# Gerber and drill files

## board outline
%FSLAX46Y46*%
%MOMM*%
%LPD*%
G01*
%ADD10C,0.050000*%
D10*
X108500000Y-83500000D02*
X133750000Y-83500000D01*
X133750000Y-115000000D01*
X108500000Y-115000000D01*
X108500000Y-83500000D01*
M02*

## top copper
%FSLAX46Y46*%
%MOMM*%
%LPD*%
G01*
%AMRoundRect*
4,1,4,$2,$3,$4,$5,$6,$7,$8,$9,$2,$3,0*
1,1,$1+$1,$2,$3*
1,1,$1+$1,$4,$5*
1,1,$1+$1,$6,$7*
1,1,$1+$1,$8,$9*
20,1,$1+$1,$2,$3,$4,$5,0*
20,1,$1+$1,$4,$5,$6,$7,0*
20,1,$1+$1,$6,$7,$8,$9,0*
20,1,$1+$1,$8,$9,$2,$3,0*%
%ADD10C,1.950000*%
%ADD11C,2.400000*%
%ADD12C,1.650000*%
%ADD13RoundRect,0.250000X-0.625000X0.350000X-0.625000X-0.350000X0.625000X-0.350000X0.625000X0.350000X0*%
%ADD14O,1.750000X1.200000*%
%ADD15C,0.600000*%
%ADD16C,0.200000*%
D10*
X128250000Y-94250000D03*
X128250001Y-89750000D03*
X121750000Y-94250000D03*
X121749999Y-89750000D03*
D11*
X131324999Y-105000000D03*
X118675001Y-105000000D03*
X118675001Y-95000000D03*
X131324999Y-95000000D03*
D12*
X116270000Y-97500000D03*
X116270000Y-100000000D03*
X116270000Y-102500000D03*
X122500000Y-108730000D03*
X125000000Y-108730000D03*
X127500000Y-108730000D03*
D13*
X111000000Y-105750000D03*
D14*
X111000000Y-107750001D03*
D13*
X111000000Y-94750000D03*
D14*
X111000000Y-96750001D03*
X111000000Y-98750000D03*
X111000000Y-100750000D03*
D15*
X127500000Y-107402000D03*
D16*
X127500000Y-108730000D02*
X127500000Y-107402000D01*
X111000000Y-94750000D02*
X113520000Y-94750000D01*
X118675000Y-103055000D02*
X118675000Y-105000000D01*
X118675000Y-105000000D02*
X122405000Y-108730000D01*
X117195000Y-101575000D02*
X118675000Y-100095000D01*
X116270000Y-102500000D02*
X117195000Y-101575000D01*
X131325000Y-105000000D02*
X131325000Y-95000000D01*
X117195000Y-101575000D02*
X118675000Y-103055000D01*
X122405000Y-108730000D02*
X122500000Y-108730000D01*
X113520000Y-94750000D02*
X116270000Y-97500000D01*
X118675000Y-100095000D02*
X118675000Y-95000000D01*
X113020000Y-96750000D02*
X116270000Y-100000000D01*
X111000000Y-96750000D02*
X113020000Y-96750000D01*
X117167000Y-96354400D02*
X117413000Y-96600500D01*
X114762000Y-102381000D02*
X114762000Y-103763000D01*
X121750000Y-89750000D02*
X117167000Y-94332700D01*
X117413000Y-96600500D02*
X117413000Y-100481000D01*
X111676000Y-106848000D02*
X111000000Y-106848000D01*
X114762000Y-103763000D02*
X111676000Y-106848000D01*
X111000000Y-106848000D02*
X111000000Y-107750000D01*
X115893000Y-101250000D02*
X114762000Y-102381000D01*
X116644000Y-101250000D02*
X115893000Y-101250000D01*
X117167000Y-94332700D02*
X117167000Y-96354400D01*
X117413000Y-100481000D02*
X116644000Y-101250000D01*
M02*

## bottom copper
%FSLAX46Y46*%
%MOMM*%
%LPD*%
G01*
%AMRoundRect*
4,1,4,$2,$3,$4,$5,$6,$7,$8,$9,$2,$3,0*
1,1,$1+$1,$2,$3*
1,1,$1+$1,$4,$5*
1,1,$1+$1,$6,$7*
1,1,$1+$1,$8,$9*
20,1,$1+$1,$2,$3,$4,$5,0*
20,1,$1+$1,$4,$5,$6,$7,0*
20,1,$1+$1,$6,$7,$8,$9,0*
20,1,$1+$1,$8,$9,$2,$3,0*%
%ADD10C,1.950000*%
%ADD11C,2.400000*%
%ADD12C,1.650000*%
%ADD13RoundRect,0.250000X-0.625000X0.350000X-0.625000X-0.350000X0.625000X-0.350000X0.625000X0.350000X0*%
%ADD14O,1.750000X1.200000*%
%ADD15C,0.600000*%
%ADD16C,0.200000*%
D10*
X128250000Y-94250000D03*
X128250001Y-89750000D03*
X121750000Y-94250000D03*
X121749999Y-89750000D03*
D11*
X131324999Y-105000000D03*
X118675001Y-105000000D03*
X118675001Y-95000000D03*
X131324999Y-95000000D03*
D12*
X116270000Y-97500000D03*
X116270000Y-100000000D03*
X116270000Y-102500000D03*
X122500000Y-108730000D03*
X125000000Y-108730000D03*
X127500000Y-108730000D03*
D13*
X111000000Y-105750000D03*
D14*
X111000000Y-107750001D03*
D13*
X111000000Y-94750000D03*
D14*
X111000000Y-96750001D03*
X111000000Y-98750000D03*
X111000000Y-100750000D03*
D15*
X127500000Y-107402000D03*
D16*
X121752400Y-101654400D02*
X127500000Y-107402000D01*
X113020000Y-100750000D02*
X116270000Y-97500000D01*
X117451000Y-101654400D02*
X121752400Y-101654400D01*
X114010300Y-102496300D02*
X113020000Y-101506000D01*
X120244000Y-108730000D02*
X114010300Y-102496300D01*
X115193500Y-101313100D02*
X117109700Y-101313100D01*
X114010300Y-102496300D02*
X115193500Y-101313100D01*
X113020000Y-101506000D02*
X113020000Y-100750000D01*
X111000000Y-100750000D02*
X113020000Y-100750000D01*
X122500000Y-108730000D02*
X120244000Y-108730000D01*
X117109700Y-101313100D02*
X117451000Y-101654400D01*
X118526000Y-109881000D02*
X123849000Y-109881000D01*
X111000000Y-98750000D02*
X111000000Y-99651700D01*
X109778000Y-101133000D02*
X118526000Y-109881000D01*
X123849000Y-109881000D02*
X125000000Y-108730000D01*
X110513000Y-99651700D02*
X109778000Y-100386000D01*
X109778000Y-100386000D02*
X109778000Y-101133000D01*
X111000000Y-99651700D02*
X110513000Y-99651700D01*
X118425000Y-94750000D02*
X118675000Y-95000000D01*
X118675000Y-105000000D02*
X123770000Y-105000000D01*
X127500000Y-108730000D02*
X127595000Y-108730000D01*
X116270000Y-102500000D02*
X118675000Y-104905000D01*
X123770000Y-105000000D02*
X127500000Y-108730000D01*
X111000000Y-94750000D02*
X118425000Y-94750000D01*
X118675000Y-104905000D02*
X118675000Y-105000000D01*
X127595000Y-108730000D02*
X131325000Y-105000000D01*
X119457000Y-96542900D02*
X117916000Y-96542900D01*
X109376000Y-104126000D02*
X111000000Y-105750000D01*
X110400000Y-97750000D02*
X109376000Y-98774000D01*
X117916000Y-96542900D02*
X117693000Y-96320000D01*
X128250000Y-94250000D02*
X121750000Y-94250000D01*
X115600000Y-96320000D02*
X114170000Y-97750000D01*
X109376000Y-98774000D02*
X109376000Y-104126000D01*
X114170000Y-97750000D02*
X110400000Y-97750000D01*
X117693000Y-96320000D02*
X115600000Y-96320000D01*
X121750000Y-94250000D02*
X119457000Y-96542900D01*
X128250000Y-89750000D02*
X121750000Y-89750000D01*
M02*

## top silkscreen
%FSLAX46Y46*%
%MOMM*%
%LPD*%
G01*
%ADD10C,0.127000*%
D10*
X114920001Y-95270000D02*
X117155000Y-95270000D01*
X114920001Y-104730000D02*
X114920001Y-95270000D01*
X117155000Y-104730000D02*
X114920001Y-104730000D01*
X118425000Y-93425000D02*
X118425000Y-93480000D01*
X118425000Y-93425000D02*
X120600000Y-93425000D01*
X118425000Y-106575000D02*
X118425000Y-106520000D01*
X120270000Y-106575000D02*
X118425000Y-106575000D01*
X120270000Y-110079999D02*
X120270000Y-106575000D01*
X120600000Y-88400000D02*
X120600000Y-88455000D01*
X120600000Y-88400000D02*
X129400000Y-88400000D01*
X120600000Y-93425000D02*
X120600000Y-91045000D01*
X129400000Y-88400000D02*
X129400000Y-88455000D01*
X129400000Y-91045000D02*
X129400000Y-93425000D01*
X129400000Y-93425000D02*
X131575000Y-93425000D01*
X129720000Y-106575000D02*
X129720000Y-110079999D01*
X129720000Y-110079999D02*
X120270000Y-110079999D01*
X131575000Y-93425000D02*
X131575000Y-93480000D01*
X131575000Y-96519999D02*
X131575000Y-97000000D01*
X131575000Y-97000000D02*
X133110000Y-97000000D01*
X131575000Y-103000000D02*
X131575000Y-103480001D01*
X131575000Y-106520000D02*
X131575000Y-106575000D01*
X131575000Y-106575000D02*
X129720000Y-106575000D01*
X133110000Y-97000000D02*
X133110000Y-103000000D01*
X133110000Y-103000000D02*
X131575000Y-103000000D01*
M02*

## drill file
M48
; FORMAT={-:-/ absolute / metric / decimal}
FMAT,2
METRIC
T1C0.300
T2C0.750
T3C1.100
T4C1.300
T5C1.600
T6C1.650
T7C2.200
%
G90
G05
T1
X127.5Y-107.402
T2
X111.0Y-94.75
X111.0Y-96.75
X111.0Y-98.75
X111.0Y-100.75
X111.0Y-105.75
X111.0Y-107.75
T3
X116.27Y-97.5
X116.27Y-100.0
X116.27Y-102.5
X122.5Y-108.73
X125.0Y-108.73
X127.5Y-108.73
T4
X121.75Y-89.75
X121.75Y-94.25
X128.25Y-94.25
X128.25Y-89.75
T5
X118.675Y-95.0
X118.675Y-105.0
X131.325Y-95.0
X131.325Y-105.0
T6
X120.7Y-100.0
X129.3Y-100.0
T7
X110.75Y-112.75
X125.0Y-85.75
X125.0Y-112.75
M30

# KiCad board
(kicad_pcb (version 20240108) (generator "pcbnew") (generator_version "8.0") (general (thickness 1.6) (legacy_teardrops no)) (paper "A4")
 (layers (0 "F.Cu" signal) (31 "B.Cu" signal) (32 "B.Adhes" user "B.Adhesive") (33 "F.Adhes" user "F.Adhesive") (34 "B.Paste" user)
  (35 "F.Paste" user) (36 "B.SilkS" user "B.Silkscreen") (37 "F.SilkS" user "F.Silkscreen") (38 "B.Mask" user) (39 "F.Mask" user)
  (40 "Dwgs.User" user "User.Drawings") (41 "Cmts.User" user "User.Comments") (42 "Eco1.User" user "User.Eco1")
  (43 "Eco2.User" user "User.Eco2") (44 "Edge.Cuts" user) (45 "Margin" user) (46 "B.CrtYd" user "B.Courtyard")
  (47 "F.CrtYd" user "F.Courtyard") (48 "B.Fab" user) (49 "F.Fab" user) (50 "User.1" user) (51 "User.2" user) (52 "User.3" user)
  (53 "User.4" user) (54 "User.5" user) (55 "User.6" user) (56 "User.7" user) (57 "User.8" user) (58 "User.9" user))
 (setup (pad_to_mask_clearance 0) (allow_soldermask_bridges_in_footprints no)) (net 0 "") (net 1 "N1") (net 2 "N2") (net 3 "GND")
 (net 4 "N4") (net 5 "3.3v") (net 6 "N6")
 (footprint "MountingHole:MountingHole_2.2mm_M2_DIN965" (layer "F.Cu") (at 110.75 112.75)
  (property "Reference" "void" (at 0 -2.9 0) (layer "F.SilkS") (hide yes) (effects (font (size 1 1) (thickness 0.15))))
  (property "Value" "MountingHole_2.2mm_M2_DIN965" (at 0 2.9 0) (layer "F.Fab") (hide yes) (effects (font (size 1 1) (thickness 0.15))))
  (pad "" np_thru_hole circle (at 0 0) (size 2.2 2.2) (drill 2.2) (layers "F&B.Cu" "*.Mask")))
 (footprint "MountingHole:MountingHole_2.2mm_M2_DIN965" (layer "F.Cu") (at 125 112.75 45)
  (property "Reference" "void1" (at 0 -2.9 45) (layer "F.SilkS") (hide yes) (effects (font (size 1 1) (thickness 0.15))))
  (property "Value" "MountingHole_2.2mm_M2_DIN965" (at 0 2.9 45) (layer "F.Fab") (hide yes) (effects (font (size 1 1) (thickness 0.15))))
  (pad "" np_thru_hole circle (at 0 0 45) (size 2.2 2.2) (drill 2.2) (layers "F&B.Cu" "*.Mask")))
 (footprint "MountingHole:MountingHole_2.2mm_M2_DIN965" (layer "F.Cu") (at 125 85.75)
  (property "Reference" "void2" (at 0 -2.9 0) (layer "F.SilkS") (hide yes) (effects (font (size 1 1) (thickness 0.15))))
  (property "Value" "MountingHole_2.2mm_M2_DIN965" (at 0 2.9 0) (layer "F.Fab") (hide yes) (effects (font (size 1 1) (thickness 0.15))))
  (pad "" np_thru_hole circle (at 0 0) (size 2.2 2.2) (drill 2.2) (layers "*.Cu" "*.Mask")))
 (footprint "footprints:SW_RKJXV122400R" (layer "F.Cu") (at 125 100 180)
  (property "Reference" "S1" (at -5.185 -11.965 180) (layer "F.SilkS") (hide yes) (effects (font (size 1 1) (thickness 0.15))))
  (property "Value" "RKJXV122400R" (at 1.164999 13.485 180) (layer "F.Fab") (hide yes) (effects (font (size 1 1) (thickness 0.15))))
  (fp_line (start 10.079999 4.73) (end 7.845 4.73) (stroke (width 0.127) (type solid)) (layer "F.SilkS"))
  (fp_line (start 10.079999 -4.73) (end 10.079999 4.73) (stroke (width 0.127) (type solid)) (layer "F.SilkS"))
  (fp_line (start 7.845 -4.73) (end 10.079999 -4.73) (stroke (width 0.127) (type solid)) (layer "F.SilkS"))
  (fp_line (start 6.575 6.575) (end 6.575 6.52) (stroke (width 0.127) (type solid)) (layer "F.SilkS"))
  (fp_line (start 6.575 6.575) (end 4.4 6.575) (stroke (width 0.127) (type solid)) (layer "F.SilkS"))
  (fp_line (start 6.575 -6.575) (end 6.575 -6.52) (stroke (width 0.127) (type solid)) (layer "F.SilkS"))
  (fp_line (start 4.73 -6.575) (end 6.575 -6.575) (stroke (width 0.127) (type solid)) (layer "F.SilkS"))
  (fp_line (start 4.73 -10.079999) (end 4.73 -6.575) (stroke (width 0.127) (type solid)) (layer "F.SilkS"))
  (fp_line (start 4.4 11.6) (end 4.4 11.545) (stroke (width 0.127) (type solid)) (layer "F.SilkS"))
  (fp_line (start 4.4 11.6) (end -4.4 11.6) (stroke (width 0.127) (type solid)) (layer "F.SilkS"))
  (fp_line (start 4.4 6.575) (end 4.4 8.955) (stroke (width 0.127) (type solid)) (layer "F.SilkS"))
  (fp_line (start -4.4 11.6) (end -4.4 11.545) (stroke (width 0.127) (type solid)) (layer "F.SilkS"))
  (fp_line (start -4.4 8.955) (end -4.4 6.575) (stroke (width 0.127) (type solid)) (layer "F.SilkS"))
  (fp_line (start -4.4 6.575) (end -6.575 6.575) (stroke (width 0.127) (type solid)) (layer "F.SilkS"))
  (fp_line (start -4.72 -6.575) (end -4.72 -10.079999) (stroke (width 0.127) (type solid)) (layer "F.SilkS"))
  (fp_line (start -4.72 -10.079999) (end 4.73 -10.079999) (stroke (width 0.127) (type solid)) (layer "F.SilkS"))
  (fp_line (start -6.575 6.575) (end -6.575 6.52) (stroke (width 0.127) (type solid)) (layer "F.SilkS"))
  (fp_line (start -6.575 3.480001) (end -6.575 3) (stroke (width 0.127) (type solid)) (layer "F.SilkS"))
  (fp_line (start -6.575 3) (end -8.11 3) (stroke (width 0.127) (type solid)) (layer "F.SilkS"))
  (fp_line (start -6.575 -3) (end -6.575 -3.480001) (stroke (width 0.127) (type solid)) (layer "F.SilkS"))
  (fp_line (start -6.575 -6.52) (end -6.575 -6.575) (stroke (width 0.127) (type solid)) (layer "F.SilkS"))
  (fp_line (start -6.575 -6.575) (end -4.72 -6.575) (stroke (width 0.127) (type solid)) (layer "F.SilkS"))
  (fp_line (start -8.11 3) (end -8.11 -3) (stroke (width 0.127) (type solid)) (layer "F.SilkS"))
  (fp_line (start -8.11 -3) (end -6.575 -3) (stroke (width 0.127) (type solid)) (layer "F.SilkS"))
  (pad "" np_thru_hole circle (at -4.3 0 180) (size 1.65 1.65) (drill 1.65) (layers "*.Cu" "*.Mask"))
  (pad "" np_thru_hole circle (at 4.3 0 180) (size 1.65 1.65) (drill 1.65) (layers "*.Cu" "*.Mask"))
  (pad "A" thru_hole circle (at -3.25 5.75 180) (size 1.95 1.95) (drill 1.3) (layers "*.Cu" "*.Mask") (remove_unused_layers no) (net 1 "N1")
   (solder_mask_margin 0.102))
  (pad "B" thru_hole circle (at -3.250001 10.25 180) (size 1.95 1.95) (drill 1.3) (layers "*.Cu" "*.Mask") (remove_unused_layers no)
   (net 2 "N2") (solder_mask_margin 0.102))
  (pad "C" thru_hole circle (at 3.25 5.75 180) (size 1.95 1.95) (drill 1.3) (layers "*.Cu" "*.Mask") (remove_unused_layers no) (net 1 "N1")
   (solder_mask_margin 0.102))
  (pad "D" thru_hole circle (at 3.250001 10.25 180) (size 1.95 1.95) (drill 1.3) (layers "*.Cu" "*.Mask") (remove_unused_layers no)
   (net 2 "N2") (solder_mask_margin 0.102))
  (pad "SH1" thru_hole circle (at -6.324999 -5 180) (size 2.4 2.4) (drill 1.6) (layers "*.Cu" "*.Mask") (remove_unused_layers no)
   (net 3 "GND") (solder_mask_margin 0.102))
  (pad "SH2" thru_hole circle (at 6.324999 -5 180) (size 2.4 2.4) (drill 1.6) (layers "*.Cu" "*.Mask") (remove_unused_layers no)
   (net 3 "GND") (solder_mask_margin 0.102))
  (pad "SH3" thru_hole circle (at 6.324999 5 180) (size 2.4 2.4) (drill 1.6) (layers "*.Cu" "*.Mask") (remove_unused_layers no)
   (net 3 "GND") (solder_mask_margin 0.102))
  (pad "SH4" thru_hole circle (at -6.324999 5 180) (size 2.4 2.4) (drill 1.6) (layers "*.Cu" "*.Mask") (remove_unused_layers no)
   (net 3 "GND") (solder_mask_margin 0.102))
  (pad "VR1_1" thru_hole circle (at 8.73 2.5 180) (size 1.65 1.65) (drill 1.1) (layers "*.Cu" "*.Mask") (remove_unused_layers no)
   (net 3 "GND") (solder_mask_margin 0.102))
  (pad "VR1_2" thru_hole circle (at 8.73 0 180) (size 1.65 1.65) (drill 1.1) (layers "*.Cu" "*.Mask") (remove_unused_layers no) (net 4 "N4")
   (solder_mask_margin 0.102))
  (pad "VR1_3" thru_hole circle (at 8.73 -2.5 180) (size 1.65 1.65) (drill 1.1) (layers "*.Cu" "*.Mask") (remove_unused_layers no)
   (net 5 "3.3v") (solder_mask_margin 0.102))
  (pad "VR2_1" thru_hole circle (at 2.5 -8.73 180) (size 1.65 1.65) (drill 1.1) (layers "*.Cu" "*.Mask") (remove_unused_layers no)
   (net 3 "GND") (solder_mask_margin 0.102))
  (pad "VR2_2" thru_hole circle (at 0 -8.73 180) (size 1.65 1.65) (drill 1.1) (layers "*.Cu" "*.Mask") (remove_unused_layers no)
   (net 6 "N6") (solder_mask_margin 0.102))
  (pad "VR2_3" thru_hole circle (at -2.5 -8.73 180) (size 1.65 1.65) (drill 1.1) (layers "*.Cu" "*.Mask") (remove_unused_layers no)
   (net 5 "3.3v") (solder_mask_margin 0.102))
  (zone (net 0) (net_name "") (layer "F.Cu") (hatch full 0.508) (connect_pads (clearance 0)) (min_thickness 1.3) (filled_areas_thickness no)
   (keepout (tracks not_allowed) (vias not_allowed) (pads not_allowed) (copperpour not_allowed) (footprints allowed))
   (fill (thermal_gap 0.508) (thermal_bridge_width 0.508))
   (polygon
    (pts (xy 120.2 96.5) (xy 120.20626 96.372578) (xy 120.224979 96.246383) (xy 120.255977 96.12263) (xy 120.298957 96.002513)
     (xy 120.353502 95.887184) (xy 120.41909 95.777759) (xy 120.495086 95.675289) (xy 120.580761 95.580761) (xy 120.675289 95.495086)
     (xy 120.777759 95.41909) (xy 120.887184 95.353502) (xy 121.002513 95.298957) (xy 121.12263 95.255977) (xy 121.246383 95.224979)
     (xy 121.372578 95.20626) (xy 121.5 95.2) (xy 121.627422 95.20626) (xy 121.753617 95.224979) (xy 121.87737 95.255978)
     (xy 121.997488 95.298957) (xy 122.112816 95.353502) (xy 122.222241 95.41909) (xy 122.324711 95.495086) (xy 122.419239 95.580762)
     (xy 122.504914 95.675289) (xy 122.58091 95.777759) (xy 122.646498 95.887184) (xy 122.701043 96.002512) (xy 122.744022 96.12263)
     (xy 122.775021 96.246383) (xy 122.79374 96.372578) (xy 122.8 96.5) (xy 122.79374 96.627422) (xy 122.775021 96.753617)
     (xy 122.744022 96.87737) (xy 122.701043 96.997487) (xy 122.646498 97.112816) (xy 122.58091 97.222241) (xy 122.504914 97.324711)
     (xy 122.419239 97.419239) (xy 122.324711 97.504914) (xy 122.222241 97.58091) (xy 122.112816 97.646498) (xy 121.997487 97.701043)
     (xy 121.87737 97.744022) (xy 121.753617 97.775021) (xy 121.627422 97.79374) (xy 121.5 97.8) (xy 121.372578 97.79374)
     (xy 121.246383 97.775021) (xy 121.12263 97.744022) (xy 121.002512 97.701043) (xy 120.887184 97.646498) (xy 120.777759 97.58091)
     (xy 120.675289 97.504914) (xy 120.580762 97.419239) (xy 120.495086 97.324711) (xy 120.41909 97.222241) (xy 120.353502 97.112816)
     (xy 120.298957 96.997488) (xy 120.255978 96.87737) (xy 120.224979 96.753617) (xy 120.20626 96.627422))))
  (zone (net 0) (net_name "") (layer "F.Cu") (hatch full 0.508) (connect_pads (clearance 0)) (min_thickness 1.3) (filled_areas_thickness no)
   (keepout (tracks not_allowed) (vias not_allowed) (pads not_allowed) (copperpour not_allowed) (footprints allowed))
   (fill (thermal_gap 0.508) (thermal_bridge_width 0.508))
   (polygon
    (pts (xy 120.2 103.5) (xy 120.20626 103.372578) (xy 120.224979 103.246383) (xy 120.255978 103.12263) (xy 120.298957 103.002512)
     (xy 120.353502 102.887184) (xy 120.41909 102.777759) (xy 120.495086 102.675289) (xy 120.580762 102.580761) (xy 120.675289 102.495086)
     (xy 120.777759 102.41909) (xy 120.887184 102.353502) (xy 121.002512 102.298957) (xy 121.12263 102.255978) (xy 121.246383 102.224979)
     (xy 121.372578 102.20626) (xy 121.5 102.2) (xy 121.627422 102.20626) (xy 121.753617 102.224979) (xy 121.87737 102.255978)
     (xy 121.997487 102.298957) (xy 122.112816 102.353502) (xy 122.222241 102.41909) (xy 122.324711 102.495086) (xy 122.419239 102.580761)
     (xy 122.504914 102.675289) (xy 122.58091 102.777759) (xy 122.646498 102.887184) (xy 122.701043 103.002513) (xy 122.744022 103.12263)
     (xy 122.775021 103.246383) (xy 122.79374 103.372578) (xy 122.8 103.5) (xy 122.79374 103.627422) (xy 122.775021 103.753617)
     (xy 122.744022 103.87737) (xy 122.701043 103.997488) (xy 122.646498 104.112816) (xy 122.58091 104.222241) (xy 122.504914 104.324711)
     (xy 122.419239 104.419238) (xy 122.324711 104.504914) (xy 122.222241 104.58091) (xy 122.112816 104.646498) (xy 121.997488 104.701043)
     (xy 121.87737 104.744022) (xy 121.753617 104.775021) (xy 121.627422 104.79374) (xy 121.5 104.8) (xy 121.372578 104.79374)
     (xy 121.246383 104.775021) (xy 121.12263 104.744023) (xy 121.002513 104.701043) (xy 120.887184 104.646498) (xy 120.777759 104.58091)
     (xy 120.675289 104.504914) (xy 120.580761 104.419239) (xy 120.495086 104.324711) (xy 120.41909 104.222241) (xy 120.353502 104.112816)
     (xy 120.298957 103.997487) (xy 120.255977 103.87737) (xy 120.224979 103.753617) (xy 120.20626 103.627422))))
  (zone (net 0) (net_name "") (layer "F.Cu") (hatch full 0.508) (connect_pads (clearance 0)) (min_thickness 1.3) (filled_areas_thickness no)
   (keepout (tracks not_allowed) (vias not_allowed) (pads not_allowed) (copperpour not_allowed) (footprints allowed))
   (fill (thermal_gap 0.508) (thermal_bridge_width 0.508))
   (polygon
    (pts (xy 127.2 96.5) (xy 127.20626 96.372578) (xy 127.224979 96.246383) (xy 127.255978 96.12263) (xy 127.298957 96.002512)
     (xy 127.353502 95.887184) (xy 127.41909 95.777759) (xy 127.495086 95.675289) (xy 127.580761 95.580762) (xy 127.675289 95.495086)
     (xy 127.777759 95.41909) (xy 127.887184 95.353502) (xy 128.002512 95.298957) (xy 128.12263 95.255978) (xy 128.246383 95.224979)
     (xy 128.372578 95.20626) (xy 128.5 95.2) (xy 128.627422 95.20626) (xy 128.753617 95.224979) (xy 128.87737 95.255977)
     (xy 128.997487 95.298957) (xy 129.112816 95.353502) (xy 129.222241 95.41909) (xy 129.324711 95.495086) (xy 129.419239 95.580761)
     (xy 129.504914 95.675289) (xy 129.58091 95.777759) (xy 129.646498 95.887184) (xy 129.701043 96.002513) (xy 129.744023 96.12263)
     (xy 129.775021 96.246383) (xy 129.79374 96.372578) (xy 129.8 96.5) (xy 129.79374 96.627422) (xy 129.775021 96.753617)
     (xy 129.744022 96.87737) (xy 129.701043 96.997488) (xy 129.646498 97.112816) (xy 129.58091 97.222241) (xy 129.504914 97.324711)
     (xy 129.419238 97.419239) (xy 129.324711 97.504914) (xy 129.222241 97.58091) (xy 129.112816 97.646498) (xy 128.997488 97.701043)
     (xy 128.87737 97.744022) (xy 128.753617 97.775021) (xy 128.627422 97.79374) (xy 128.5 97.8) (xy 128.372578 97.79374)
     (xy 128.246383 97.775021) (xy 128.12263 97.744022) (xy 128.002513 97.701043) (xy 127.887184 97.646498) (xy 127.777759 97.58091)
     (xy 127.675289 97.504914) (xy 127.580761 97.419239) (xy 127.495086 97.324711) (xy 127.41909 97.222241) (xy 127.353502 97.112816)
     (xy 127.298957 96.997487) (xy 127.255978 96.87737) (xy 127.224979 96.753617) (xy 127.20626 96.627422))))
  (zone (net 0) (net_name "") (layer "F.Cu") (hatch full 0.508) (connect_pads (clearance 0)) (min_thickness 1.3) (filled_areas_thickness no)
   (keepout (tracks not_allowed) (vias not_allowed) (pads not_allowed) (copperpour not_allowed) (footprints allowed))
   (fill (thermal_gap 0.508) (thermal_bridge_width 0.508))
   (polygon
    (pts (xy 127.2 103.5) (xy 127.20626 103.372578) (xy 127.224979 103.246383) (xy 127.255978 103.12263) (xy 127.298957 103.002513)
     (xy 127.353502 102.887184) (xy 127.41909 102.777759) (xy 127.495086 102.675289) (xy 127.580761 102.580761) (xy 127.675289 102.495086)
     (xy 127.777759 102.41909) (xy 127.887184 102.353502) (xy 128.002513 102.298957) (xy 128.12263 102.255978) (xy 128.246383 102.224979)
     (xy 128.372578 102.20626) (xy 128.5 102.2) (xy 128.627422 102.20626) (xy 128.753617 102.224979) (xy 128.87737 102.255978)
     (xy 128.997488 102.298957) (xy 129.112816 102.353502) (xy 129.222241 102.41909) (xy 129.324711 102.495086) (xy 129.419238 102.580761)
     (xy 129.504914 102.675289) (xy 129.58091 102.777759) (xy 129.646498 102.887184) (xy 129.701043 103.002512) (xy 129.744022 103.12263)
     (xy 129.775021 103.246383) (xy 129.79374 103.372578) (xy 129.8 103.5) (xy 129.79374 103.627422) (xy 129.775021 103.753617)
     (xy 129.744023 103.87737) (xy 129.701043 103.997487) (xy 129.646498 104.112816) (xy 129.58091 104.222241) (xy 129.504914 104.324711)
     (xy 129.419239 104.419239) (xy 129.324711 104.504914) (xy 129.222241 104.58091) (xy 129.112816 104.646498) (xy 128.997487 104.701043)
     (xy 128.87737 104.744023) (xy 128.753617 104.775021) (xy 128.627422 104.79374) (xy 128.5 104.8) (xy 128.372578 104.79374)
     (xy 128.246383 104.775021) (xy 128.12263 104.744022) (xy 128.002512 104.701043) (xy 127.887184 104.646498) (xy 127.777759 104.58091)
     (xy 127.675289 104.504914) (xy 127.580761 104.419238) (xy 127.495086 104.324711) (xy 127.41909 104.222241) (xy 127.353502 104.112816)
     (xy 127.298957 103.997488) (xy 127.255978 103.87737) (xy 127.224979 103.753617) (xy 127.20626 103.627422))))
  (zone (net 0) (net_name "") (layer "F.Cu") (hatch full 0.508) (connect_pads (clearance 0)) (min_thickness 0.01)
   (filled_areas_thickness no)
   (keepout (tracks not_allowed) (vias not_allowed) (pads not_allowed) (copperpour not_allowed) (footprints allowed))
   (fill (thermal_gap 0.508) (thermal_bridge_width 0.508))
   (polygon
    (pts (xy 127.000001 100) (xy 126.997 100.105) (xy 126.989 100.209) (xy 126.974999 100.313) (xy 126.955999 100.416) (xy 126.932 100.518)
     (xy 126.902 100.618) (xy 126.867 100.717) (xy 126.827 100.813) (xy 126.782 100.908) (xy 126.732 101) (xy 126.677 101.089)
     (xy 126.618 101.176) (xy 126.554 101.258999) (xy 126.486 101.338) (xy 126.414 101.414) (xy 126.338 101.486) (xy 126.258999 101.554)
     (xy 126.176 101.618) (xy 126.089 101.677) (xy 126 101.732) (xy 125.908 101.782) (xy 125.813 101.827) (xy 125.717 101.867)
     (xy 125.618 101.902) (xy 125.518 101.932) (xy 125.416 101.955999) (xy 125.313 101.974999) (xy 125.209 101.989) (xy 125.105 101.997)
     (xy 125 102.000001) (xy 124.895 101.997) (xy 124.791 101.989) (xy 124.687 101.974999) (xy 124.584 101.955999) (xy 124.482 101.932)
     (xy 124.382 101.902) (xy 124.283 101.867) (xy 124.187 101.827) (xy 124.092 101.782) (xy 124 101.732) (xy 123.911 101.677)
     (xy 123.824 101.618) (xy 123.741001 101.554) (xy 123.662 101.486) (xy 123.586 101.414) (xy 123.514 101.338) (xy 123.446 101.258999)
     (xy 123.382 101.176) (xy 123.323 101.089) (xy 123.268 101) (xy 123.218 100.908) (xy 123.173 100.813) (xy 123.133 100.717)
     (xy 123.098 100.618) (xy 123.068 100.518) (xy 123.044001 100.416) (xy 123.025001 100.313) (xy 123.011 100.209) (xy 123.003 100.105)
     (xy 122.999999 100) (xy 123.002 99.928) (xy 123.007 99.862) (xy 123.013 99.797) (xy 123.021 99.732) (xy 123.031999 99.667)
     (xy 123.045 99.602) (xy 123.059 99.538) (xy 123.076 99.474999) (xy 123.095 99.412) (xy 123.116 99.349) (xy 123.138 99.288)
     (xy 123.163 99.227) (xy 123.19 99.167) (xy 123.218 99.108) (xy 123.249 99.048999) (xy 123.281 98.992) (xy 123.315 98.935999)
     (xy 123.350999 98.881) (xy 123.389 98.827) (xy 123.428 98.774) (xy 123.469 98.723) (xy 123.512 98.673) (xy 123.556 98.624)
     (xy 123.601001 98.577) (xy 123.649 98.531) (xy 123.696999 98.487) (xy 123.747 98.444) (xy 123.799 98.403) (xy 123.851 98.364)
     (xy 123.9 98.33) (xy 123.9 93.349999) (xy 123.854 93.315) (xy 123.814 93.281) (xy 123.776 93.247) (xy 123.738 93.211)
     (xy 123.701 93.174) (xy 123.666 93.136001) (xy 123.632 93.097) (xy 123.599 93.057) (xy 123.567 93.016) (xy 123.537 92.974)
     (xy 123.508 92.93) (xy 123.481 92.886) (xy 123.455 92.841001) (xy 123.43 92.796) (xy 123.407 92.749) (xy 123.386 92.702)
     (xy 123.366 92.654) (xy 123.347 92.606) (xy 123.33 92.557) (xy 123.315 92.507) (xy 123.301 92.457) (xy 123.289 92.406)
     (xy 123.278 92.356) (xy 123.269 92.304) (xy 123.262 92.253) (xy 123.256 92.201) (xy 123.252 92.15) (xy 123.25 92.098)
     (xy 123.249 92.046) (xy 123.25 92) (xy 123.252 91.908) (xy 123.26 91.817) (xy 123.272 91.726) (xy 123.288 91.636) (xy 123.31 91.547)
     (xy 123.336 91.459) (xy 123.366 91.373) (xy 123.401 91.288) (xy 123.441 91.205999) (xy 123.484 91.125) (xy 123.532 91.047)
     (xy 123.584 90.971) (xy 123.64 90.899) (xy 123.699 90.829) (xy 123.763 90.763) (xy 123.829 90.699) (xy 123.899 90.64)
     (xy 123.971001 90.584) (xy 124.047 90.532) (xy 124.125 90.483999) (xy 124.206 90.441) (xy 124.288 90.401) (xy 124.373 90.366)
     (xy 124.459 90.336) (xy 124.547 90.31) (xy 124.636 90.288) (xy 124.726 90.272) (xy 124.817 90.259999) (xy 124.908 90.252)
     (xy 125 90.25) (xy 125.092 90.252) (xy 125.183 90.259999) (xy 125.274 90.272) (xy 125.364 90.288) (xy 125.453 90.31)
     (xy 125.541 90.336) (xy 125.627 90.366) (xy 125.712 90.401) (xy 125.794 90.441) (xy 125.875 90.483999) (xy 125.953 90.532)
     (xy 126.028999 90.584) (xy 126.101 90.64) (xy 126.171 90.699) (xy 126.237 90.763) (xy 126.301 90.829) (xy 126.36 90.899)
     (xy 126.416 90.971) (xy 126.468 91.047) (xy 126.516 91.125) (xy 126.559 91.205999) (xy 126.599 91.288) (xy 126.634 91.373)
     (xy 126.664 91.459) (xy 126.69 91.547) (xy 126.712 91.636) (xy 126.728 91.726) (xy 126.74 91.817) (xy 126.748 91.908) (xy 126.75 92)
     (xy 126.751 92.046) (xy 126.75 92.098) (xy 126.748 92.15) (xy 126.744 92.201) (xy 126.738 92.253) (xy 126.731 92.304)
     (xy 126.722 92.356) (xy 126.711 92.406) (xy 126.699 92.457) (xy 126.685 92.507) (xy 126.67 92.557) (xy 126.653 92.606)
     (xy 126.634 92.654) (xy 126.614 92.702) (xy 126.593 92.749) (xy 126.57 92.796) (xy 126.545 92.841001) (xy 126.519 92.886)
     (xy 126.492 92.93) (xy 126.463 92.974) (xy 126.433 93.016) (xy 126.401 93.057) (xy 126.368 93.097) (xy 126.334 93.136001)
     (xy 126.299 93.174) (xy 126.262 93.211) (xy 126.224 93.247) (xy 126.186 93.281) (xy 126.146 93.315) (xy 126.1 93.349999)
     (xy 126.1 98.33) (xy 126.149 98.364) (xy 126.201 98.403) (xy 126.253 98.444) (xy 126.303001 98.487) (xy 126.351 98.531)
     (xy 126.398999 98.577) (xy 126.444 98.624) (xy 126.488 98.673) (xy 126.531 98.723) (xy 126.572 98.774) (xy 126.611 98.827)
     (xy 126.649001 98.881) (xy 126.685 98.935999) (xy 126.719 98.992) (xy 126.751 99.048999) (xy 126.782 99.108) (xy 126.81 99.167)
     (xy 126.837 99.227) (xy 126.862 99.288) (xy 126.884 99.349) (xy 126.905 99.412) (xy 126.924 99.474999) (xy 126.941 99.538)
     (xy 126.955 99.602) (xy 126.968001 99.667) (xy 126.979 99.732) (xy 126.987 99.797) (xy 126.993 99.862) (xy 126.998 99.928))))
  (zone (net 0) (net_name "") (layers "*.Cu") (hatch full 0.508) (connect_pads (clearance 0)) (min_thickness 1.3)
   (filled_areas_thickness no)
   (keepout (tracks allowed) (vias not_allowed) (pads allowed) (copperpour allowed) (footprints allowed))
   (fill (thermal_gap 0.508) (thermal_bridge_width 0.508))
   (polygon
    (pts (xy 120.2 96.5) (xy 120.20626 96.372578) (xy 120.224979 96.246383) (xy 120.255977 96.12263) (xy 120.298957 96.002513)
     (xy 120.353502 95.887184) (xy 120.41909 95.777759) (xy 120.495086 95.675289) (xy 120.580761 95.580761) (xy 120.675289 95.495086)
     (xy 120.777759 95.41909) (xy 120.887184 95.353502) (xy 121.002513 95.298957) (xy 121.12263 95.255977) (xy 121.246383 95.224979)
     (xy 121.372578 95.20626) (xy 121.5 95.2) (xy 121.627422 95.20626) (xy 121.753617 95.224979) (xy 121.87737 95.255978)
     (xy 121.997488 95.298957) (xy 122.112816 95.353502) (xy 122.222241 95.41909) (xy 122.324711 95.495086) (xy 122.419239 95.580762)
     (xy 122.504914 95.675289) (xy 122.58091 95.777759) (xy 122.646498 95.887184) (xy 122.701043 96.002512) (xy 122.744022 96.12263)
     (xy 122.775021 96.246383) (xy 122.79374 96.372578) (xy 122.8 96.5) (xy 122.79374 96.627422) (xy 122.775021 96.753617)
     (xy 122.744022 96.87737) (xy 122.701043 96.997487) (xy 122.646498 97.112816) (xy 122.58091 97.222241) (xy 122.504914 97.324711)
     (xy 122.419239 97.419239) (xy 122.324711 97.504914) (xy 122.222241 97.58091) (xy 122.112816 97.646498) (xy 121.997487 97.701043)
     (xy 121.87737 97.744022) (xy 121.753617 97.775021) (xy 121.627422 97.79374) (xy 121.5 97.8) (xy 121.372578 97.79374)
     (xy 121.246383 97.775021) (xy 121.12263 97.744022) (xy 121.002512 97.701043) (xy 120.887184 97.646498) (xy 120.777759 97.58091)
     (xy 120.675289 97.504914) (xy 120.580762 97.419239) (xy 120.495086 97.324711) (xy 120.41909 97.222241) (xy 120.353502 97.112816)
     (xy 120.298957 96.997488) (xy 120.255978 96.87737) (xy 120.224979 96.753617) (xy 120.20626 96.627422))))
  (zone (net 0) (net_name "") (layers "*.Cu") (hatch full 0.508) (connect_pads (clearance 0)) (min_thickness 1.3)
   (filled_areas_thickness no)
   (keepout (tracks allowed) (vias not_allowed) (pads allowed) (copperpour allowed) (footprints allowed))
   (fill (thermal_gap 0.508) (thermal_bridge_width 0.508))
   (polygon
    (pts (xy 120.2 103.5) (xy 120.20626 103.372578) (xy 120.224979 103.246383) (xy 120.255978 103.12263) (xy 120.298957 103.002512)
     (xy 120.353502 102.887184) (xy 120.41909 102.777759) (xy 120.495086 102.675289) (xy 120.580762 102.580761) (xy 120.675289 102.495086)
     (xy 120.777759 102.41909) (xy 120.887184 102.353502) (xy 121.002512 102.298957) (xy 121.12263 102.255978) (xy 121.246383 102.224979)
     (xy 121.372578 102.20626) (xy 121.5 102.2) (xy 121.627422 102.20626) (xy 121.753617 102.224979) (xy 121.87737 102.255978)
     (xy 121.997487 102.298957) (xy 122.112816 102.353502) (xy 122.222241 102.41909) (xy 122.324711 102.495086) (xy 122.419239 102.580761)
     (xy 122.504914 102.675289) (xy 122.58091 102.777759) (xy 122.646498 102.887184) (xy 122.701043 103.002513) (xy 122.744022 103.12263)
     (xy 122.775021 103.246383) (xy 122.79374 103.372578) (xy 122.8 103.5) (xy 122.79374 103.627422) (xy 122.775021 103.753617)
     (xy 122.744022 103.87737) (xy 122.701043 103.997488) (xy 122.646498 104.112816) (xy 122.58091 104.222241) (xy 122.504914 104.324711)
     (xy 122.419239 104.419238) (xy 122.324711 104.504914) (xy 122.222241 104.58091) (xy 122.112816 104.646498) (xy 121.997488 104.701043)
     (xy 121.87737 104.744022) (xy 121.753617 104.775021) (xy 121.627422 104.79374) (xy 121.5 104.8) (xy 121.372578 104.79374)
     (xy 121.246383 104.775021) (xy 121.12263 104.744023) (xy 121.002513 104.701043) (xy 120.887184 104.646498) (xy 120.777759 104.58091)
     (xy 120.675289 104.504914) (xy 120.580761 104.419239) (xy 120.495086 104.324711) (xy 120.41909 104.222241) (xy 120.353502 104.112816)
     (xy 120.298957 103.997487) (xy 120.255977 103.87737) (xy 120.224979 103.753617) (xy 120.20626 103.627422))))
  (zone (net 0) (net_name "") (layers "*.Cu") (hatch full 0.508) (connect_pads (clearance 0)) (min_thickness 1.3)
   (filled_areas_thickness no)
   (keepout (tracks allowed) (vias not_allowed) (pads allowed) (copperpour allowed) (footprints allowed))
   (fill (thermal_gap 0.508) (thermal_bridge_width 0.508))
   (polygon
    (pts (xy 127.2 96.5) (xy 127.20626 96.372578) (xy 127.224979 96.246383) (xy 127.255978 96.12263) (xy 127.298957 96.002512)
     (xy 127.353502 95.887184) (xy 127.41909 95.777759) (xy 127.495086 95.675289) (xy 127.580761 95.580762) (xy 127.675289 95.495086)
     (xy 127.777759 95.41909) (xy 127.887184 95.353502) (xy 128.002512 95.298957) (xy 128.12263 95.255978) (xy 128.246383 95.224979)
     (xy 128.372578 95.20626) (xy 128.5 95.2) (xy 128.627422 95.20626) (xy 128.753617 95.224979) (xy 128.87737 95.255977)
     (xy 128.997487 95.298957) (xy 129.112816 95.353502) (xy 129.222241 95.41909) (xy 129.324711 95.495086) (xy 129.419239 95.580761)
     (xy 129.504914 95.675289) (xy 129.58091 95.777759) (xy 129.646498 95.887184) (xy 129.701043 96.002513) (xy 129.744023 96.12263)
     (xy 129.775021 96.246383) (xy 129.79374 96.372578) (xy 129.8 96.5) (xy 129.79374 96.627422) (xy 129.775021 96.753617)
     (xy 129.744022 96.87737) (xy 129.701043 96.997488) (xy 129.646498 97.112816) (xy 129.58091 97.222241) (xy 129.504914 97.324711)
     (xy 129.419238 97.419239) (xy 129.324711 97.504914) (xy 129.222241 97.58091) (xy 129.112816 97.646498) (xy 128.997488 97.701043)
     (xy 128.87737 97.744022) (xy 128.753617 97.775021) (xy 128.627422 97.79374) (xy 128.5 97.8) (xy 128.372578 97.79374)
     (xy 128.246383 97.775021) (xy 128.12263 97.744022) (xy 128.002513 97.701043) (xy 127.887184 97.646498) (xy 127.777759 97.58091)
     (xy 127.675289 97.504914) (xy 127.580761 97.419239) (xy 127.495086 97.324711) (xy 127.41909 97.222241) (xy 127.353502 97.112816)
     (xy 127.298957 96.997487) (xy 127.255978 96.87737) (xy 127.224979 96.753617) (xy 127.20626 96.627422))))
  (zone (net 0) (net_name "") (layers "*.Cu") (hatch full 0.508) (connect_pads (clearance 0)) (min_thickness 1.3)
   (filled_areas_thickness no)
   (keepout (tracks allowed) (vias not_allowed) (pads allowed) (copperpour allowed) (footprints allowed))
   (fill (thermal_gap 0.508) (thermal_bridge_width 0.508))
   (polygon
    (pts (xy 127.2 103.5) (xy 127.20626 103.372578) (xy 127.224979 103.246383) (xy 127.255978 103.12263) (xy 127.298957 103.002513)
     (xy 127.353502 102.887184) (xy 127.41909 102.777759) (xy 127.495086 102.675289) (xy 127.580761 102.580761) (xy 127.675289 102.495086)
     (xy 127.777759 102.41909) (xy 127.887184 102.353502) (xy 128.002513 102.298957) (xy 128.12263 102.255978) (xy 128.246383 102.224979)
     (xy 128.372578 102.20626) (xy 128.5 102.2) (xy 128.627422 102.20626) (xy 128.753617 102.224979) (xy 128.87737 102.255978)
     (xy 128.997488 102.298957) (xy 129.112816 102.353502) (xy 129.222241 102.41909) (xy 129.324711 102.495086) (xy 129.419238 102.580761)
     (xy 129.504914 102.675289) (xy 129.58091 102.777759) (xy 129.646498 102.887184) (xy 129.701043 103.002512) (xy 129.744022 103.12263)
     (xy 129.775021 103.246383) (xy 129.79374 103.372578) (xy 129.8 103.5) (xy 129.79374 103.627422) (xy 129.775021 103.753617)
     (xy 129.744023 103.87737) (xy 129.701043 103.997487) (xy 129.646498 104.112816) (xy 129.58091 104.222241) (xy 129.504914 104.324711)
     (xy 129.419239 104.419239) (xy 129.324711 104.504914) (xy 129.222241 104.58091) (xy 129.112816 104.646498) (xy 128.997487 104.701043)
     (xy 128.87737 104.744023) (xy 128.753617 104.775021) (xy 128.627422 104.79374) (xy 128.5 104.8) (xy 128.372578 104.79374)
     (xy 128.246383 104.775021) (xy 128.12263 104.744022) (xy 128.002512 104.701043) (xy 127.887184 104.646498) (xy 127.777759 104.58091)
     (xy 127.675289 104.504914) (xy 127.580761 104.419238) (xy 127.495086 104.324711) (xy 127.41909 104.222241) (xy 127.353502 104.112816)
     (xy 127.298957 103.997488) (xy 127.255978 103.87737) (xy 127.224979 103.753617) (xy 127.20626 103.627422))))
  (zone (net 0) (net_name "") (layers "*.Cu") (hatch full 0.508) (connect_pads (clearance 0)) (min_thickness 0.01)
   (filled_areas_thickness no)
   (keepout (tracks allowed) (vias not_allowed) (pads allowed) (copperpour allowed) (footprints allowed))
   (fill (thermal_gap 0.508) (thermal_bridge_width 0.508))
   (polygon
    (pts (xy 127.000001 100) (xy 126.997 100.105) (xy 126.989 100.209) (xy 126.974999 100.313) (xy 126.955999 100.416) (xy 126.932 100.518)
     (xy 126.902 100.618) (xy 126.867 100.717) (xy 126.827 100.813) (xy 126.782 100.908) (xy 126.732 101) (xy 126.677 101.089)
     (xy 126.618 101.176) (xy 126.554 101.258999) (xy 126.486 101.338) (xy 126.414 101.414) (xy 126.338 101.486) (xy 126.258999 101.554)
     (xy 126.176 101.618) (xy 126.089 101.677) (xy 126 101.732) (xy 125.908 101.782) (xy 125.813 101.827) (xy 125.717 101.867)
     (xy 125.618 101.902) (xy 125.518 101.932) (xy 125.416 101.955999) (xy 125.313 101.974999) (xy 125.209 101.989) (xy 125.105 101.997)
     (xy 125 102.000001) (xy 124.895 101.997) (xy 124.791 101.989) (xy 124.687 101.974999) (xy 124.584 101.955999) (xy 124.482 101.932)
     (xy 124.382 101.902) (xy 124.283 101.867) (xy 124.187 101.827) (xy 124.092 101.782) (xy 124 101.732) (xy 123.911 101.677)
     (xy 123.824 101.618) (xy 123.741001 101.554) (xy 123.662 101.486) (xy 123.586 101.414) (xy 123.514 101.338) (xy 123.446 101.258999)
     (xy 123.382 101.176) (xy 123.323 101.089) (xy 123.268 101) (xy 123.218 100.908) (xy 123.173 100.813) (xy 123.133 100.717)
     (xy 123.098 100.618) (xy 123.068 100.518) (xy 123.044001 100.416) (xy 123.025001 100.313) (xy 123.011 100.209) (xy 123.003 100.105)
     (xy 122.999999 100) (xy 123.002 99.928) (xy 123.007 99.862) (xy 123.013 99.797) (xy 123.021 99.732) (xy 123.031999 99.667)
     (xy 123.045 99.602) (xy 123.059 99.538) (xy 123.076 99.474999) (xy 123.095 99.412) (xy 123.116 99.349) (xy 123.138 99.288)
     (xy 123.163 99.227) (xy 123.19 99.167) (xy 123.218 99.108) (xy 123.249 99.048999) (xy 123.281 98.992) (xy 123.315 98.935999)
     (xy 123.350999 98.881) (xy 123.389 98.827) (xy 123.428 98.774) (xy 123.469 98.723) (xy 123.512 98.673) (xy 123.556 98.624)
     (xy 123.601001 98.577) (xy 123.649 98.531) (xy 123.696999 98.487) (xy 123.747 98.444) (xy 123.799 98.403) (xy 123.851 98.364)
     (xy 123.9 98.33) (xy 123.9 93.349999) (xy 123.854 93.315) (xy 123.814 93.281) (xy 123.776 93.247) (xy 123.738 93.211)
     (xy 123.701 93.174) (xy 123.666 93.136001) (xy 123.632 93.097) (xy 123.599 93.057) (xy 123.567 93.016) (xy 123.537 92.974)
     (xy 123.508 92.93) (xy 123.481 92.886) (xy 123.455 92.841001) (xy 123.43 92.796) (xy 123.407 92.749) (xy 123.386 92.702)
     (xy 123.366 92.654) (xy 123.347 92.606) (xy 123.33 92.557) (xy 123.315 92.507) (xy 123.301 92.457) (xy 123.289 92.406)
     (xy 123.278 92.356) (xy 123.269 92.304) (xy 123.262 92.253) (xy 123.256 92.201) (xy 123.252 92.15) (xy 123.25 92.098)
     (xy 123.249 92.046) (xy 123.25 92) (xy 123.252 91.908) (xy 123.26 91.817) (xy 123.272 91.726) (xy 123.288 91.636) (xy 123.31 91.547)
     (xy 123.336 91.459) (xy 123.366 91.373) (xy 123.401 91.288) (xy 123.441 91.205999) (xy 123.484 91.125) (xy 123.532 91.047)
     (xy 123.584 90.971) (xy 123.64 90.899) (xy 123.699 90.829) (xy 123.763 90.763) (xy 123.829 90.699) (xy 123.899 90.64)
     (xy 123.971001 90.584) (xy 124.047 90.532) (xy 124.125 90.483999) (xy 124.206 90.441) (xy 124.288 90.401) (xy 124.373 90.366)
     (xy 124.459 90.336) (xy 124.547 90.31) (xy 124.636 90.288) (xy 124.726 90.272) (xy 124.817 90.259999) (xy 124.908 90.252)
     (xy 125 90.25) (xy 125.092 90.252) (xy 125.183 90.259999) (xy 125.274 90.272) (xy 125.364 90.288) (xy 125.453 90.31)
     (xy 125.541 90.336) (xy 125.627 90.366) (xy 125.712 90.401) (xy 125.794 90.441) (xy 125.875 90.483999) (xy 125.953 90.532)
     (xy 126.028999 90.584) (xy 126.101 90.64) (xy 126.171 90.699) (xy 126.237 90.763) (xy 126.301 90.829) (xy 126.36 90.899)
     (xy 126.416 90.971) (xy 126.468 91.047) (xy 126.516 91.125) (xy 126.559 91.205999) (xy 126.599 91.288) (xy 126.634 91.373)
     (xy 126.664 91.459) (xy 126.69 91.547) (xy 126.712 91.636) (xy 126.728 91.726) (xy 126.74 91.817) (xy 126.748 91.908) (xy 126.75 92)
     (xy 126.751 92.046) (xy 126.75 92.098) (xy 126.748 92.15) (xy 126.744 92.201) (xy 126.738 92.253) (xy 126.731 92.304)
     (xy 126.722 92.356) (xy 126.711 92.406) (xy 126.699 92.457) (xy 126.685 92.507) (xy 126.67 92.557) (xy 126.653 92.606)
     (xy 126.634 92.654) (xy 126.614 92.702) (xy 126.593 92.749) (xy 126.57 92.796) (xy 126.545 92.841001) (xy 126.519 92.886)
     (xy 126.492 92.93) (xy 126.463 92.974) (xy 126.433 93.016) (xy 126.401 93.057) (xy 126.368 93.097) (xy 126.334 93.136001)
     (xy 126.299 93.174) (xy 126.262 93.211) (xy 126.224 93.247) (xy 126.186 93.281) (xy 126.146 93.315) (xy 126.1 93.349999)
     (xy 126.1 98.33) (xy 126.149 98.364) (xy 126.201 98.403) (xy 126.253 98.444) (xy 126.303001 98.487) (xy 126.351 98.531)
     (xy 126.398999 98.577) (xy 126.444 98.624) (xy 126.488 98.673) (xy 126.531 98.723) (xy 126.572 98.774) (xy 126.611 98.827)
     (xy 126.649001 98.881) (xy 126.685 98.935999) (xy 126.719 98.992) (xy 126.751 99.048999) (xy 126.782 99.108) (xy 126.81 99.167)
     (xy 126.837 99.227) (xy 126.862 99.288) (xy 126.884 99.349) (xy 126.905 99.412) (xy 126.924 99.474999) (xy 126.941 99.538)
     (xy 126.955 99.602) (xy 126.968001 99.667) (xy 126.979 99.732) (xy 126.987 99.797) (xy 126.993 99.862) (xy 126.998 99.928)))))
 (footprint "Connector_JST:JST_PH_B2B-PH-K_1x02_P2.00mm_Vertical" (layer "B.Cu") (at 111 105.75 -90)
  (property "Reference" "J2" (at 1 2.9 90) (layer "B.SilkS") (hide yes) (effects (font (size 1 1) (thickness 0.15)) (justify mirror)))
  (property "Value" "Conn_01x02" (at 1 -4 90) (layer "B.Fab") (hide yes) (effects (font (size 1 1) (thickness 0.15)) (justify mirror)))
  (pad "1" thru_hole roundrect (at 0 0 270) (size 1.2 1.75) (drill 0.75) (layers "*.Cu" "*.Mask") (remove_unused_layers no)
   (roundrect_rratio 0.208333) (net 1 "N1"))
  (pad "2" thru_hole oval (at 2.000001 0 270) (size 1.2 1.75) (drill 0.75) (layers "*.Cu" "*.Mask") (remove_unused_layers no) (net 2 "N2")))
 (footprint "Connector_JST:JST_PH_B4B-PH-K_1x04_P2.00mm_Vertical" (layer "B.Cu") (at 111 94.75 -90)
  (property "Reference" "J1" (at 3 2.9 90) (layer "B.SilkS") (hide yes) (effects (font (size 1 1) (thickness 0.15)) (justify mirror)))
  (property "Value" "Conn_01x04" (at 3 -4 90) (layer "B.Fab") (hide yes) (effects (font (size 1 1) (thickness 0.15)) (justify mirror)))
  (pad "1" thru_hole roundrect (at 0 0 270) (size 1.2 1.75) (drill 0.75) (layers "*.Cu" "*.Mask") (remove_unused_layers no)
   (roundrect_rratio 0.208333) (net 3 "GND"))
  (pad "2" thru_hole oval (at 2.000001 0 270) (size 1.2 1.75) (drill 0.75) (layers "*.Cu" "*.Mask") (remove_unused_layers no) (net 4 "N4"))
  (pad "3" thru_hole oval (at 4 0 270) (size 1.2 1.75) (drill 0.75) (layers "*.Cu" "*.Mask") (remove_unused_layers no) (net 6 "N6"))
  (pad "4" thru_hole oval (at 6 0 270) (size 1.2 1.75) (drill 0.75) (layers "*.Cu" "*.Mask") (remove_unused_layers no) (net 5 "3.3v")))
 (gr_rect (start 108.5 83.5) (end 133.75 115) (stroke (width 0.05) (type default)) (fill none) (layer "Edge.Cuts"))
 (segment (start 127.5 108.73) (end 127.5 107.402) (width 0.2) (layer "F.Cu") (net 5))
 (via (at 127.5 107.402) (size 0.6) (drill 0.3) (layers "F.Cu" "B.Cu") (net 5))
 (segment (start 121.7524 101.6544) (end 127.5 107.402) (width 0.2) (layer "B.Cu") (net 5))
 (segment (start 113.02 100.75) (end 116.27 97.5) (width 0.2) (layer "B.Cu") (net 5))
 (segment (start 117.451 101.6544) (end 121.7524 101.6544) (width 0.2) (layer "B.Cu") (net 5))
 (segment (start 114.0103 102.4963) (end 113.02 101.506) (width 0.2) (layer "B.Cu") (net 5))
 (segment (start 120.244 108.73) (end 114.0103 102.4963) (width 0.2) (layer "B.Cu") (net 5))
 (segment (start 115.1935 101.3131) (end 117.1097 101.3131) (width 0.2) (layer "B.Cu") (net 5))
 (segment (start 114.0103 102.4963) (end 115.1935 101.3131) (width 0.2) (layer "B.Cu") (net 5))
 (segment (start 113.02 101.506) (end 113.02 100.75) (width 0.2) (layer "B.Cu") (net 5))
 (segment (start 111 100.75) (end 113.02 100.75) (width 0.2) (layer "B.Cu") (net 5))
 (segment (start 122.5 108.73) (end 120.244 108.73) (width 0.2) (layer "B.Cu") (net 5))
 (segment (start 117.1097 101.3131) (end 117.451 101.6544) (width 0.2) (layer "B.Cu") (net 5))
 (segment (start 118.526 109.881) (end 123.849 109.881) (width 0.2) (layer "B.Cu") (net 6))
 (segment (start 111 98.75) (end 111 99.6517) (width 0.2) (layer "B.Cu") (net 6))
 (segment (start 109.778 101.133) (end 118.526 109.881) (width 0.2) (layer "B.Cu") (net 6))
 (segment (start 123.849 109.881) (end 125 108.73) (width 0.2) (layer "B.Cu") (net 6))
 (segment (start 110.513 99.6517) (end 109.778 100.386) (width 0.2) (layer "B.Cu") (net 6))
 (segment (start 109.778 100.386) (end 109.778 101.133) (width 0.2) (layer "B.Cu") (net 6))
 (segment (start 111 99.6517) (end 110.513 99.6517) (width 0.2) (layer "B.Cu") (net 6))
 (segment (start 111 94.75) (end 113.52 94.75) (width 0.2) (layer "F.Cu") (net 3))
 (segment (start 118.675 103.055) (end 118.675 105) (width 0.2) (layer "F.Cu") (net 3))
 (segment (start 118.675 105) (end 122.405 108.73) (width 0.2) (layer "F.Cu") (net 3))
 (segment (start 117.195 101.575) (end 118.675 100.095) (width 0.2) (layer "F.Cu") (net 3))
 (segment (start 116.27 102.5) (end 117.195 101.575) (width 0.2) (layer "F.Cu") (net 3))
 (segment (start 131.325 105) (end 131.325 95) (width 0.2) (layer "F.Cu") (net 3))
 (segment (start 117.195 101.575) (end 118.675 103.055) (width 0.2) (layer "F.Cu") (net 3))
 (segment (start 122.405 108.73) (end 122.5 108.73) (width 0.2) (layer "F.Cu") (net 3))
 (segment (start 113.52 94.75) (end 116.27 97.5) (width 0.2) (layer "F.Cu") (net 3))
 (segment (start 118.675 100.095) (end 118.675 95) (width 0.2) (layer "F.Cu") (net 3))
 (segment (start 118.425 94.75) (end 118.675 95) (width 0.2) (layer "B.Cu") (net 3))
 (segment (start 118.675 105) (end 123.77 105) (width 0.2) (layer "B.Cu") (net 3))
 (segment (start 127.5 108.73) (end 127.595 108.73) (width 0.2) (layer "B.Cu") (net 3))
 (segment (start 116.27 102.5) (end 118.675 104.905) (width 0.2) (layer "B.Cu") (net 3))
 (segment (start 123.77 105) (end 127.5 108.73) (width 0.2) (layer "B.Cu") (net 3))
 (segment (start 111 94.75) (end 118.425 94.75) (width 0.2) (layer "B.Cu") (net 3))
 (segment (start 118.675 104.905) (end 118.675 105) (width 0.2) (layer "B.Cu") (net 3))
 (segment (start 127.595 108.73) (end 131.325 105) (width 0.2) (layer "B.Cu") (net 3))
 (segment (start 113.02 96.75) (end 116.27 100) (width 0.2) (layer "F.Cu") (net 4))
 (segment (start 111 96.75) (end 113.02 96.75) (width 0.2) (layer "F.Cu") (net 4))
 (segment (start 119.457 96.5429) (end 117.916 96.5429) (width 0.2) (layer "B.Cu") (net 1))
 (segment (start 109.376 104.126) (end 111 105.75) (width 0.2) (layer "B.Cu") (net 1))
 (segment (start 110.4 97.75) (end 109.376 98.774) (width 0.2) (layer "B.Cu") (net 1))
 (segment (start 117.916 96.5429) (end 117.693 96.32) (width 0.2) (layer "B.Cu") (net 1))
 (segment (start 128.25 94.25) (end 121.75 94.25) (width 0.2) (layer "B.Cu") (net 1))
 (segment (start 115.6 96.32) (end 114.17 97.75) (width 0.2) (layer "B.Cu") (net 1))
 (segment (start 109.376 98.774) (end 109.376 104.126) (width 0.2) (layer "B.Cu") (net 1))
 (segment (start 114.17 97.75) (end 110.4 97.75) (width 0.2) (layer "B.Cu") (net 1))
 (segment (start 117.693 96.32) (end 115.6 96.32) (width 0.2) (layer "B.Cu") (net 1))
 (segment (start 121.75 94.25) (end 119.457 96.5429) (width 0.2) (layer "B.Cu") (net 1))
 (segment (start 117.167 96.3544) (end 117.413 96.6005) (width 0.2) (layer "F.Cu") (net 2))
 (segment (start 114.762 102.381) (end 114.762 103.763) (width 0.2) (layer "F.Cu") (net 2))
 (segment (start 121.75 89.75) (end 117.167 94.3327) (width 0.2) (layer "F.Cu") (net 2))
 (segment (start 117.413 96.6005) (end 117.413 100.481) (width 0.2) (layer "F.Cu") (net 2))
 (segment (start 111.676 106.848) (end 111 106.848) (width 0.2) (layer "F.Cu") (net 2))
 (segment (start 114.762 103.763) (end 111.676 106.848) (width 0.2) (layer "F.Cu") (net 2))
 (segment (start 111 106.848) (end 111 107.75) (width 0.2) (layer "F.Cu") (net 2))
 (segment (start 115.893 101.25) (end 114.762 102.381) (width 0.2) (layer "F.Cu") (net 2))
 (segment (start 116.644 101.25) (end 115.893 101.25) (width 0.2) (layer "F.Cu") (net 2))
 (segment (start 117.167 94.3327) (end 117.167 96.3544) (width 0.2) (layer "F.Cu") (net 2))
 (segment (start 117.413 100.481) (end 116.644 101.25) (width 0.2) (layer "F.Cu") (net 2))
 (segment (start 128.25 89.75) (end 121.75 89.75) (width 0.2) (layer "B.Cu") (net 2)))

